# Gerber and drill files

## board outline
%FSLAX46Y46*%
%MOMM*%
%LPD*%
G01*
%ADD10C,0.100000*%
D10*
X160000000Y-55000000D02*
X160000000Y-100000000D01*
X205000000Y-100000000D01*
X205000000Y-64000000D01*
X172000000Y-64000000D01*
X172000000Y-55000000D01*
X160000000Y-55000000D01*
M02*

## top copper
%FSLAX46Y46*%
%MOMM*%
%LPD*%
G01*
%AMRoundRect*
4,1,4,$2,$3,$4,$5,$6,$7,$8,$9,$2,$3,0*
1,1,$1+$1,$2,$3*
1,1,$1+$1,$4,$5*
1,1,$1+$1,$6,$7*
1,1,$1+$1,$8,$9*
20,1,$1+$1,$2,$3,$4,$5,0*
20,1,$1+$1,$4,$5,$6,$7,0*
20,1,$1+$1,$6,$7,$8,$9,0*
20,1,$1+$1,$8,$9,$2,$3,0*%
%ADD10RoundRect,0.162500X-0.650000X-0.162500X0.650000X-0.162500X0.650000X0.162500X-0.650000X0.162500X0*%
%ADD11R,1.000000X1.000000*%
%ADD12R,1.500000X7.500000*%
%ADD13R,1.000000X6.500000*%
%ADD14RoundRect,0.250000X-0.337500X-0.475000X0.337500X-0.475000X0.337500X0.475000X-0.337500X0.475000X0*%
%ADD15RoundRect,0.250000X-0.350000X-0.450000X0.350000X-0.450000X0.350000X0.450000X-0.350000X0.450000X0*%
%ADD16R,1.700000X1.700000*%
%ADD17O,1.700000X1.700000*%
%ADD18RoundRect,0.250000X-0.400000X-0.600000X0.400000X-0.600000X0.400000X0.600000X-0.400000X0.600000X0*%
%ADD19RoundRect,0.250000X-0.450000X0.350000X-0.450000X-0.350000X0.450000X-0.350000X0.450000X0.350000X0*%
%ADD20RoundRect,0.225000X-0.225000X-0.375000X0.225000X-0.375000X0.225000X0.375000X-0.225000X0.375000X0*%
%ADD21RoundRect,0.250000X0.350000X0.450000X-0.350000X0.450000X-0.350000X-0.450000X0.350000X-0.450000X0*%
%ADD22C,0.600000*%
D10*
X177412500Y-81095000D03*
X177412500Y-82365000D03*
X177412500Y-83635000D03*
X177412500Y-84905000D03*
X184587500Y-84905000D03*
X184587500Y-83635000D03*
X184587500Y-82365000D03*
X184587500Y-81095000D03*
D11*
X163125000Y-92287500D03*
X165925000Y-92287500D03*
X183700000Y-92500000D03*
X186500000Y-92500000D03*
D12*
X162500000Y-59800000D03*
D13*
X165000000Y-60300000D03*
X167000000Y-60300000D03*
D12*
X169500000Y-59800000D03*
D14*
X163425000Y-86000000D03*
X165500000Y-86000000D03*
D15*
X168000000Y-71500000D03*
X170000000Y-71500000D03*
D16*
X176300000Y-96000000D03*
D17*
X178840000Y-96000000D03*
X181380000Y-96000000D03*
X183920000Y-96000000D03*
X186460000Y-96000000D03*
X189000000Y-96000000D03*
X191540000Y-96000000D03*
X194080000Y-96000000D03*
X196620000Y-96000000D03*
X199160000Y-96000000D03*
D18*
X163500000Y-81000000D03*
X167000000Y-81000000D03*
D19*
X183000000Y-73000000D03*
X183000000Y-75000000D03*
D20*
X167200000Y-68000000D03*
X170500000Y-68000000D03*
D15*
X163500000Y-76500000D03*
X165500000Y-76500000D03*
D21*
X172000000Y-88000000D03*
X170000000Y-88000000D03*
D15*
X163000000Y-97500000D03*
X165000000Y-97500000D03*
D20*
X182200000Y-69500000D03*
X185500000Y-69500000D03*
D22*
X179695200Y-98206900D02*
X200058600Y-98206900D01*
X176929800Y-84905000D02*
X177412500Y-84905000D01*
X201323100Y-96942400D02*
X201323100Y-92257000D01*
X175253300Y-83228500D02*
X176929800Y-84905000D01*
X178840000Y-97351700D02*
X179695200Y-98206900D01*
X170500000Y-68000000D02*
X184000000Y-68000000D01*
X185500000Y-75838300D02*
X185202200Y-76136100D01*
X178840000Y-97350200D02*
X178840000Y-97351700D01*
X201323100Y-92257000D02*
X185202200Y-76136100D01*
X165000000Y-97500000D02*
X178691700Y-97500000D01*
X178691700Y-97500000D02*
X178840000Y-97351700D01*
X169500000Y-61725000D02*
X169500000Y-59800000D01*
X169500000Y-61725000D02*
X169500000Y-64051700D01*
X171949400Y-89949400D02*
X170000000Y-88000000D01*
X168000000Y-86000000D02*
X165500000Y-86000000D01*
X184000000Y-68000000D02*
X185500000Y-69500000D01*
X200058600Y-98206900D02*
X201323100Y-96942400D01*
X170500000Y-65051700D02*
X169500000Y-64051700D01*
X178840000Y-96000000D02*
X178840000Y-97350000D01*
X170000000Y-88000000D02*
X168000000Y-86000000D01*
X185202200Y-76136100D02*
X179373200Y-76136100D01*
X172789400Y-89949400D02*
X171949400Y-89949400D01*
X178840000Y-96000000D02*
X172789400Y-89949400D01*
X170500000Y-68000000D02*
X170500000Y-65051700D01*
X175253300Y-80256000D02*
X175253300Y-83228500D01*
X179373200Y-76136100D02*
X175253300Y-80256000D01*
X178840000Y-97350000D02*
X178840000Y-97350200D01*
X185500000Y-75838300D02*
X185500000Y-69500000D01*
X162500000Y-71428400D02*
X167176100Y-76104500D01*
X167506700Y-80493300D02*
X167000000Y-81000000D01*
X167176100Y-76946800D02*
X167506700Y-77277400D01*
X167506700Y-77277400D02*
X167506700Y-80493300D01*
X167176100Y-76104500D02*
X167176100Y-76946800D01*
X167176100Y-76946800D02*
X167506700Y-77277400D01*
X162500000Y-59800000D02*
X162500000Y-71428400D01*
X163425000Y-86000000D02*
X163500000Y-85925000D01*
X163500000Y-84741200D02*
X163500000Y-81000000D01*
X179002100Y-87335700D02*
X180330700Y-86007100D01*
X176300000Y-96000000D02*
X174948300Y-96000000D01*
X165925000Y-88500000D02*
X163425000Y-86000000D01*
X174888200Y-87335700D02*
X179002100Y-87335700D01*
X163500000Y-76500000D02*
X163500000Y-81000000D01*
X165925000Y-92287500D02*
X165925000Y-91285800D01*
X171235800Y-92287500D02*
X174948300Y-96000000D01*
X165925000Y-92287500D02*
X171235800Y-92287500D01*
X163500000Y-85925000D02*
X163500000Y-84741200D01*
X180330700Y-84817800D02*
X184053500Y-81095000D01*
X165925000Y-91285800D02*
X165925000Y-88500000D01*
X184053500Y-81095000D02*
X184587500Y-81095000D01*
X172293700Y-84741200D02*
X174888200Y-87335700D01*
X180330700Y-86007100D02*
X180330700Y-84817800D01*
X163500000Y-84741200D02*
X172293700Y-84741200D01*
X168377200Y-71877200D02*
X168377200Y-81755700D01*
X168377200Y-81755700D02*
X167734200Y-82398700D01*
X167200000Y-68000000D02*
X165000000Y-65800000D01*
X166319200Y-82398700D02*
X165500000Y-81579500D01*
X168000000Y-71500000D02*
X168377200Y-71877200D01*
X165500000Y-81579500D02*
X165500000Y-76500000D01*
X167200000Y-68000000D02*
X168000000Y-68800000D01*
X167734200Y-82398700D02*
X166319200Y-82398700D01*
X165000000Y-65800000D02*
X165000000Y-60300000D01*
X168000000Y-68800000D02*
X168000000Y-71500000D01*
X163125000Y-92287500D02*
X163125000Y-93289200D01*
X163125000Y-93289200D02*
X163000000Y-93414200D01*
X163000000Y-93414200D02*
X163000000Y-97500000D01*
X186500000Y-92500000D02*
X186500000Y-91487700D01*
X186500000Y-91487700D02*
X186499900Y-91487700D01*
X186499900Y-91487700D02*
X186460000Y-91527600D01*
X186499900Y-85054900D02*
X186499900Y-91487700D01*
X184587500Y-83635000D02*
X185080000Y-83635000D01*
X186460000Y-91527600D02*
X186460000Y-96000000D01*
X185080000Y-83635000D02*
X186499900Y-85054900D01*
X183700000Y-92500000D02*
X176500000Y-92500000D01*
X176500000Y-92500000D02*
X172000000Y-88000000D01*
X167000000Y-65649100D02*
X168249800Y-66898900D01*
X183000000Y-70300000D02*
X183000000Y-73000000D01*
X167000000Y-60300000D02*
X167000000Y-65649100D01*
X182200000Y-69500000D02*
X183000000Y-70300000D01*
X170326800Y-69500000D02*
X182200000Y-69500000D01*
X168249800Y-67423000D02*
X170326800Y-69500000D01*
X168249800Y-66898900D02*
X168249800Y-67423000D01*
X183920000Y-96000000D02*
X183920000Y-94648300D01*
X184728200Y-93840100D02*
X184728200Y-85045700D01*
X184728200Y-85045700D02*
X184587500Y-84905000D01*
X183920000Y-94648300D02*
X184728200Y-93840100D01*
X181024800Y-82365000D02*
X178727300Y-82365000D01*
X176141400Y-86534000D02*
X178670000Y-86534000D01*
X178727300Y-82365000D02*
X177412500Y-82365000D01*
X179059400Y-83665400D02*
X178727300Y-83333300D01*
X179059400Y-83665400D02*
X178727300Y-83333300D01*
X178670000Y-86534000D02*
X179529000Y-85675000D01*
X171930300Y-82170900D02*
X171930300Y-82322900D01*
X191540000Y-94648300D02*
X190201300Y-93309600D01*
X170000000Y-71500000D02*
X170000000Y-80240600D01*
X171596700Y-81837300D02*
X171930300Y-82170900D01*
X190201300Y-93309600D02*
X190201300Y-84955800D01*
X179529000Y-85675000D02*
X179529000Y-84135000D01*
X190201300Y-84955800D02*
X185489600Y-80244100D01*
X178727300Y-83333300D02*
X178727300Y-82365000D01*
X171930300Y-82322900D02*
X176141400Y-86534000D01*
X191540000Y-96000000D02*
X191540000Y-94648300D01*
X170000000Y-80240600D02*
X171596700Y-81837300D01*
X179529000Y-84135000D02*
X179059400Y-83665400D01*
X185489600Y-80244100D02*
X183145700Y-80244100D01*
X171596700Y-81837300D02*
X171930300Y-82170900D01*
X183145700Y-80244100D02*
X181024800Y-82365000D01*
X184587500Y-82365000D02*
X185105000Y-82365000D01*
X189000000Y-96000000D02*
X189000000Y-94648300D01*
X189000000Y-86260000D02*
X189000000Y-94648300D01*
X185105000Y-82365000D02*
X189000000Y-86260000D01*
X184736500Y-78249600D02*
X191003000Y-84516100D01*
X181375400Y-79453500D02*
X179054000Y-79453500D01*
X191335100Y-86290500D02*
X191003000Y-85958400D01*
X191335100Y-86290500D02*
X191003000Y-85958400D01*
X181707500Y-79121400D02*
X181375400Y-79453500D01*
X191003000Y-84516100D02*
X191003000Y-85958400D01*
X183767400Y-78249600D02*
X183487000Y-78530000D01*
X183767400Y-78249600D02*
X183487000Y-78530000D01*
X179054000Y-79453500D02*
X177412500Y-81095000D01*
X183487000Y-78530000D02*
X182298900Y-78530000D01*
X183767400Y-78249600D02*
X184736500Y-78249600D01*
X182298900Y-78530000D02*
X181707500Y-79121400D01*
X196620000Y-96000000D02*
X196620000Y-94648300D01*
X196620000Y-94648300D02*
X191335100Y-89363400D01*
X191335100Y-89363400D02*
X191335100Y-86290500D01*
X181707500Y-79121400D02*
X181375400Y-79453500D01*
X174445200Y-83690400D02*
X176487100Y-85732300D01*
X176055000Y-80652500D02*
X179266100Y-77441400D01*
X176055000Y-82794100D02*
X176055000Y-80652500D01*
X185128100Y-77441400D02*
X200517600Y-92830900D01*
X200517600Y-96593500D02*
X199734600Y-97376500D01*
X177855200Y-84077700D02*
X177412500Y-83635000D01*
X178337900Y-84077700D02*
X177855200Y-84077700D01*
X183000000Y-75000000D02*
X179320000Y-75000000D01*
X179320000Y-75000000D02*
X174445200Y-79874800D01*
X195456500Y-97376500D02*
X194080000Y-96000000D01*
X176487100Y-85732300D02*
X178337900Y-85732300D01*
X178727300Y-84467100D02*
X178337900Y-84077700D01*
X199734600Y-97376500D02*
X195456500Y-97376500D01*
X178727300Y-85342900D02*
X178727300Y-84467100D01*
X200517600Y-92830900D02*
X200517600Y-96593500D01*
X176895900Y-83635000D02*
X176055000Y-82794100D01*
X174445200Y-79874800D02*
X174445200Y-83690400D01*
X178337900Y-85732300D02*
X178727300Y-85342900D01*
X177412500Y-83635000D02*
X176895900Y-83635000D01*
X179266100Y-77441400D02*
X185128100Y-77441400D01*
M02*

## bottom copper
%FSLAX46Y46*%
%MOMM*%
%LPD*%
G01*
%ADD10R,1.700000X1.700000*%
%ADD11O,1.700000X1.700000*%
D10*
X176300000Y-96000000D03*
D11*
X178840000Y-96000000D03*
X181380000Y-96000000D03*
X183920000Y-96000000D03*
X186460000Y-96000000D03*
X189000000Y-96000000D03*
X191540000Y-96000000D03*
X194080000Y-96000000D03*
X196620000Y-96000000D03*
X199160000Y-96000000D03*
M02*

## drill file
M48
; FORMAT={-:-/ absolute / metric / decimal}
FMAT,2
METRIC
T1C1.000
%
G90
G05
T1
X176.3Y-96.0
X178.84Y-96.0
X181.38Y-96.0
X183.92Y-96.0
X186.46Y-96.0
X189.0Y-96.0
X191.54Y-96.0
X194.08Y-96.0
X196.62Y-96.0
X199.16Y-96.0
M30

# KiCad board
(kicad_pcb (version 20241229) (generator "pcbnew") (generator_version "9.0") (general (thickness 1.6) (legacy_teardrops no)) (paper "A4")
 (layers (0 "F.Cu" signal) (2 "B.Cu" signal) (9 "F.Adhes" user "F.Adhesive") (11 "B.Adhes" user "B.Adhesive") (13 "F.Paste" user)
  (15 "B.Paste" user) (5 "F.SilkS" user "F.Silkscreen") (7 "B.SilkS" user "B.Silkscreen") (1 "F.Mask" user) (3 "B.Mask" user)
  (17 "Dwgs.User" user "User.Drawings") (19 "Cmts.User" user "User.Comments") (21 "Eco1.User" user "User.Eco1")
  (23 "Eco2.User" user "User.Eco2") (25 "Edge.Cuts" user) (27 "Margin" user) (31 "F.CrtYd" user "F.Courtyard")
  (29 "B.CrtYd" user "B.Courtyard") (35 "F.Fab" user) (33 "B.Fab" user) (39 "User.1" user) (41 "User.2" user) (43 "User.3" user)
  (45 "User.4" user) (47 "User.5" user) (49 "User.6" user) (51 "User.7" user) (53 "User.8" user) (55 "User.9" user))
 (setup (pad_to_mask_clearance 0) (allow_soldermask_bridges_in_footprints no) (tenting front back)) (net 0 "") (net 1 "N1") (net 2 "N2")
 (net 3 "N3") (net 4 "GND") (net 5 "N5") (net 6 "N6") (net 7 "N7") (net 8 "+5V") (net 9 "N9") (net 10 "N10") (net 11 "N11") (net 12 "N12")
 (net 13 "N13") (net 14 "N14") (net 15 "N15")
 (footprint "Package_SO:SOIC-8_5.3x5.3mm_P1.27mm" (layer "F.Cu") (at 181 83)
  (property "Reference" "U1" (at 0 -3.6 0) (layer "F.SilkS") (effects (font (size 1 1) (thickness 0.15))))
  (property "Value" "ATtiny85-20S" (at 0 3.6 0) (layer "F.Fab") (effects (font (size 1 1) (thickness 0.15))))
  (pad "1" smd roundrect (at -3.5875 -1.905) (size 1.625 0.65) (layers "F.Cu" "F.Mask" "F.Paste") (roundrect_rratio 0.25) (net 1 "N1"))
  (pad "2" smd roundrect (at -3.5875 -0.635) (size 1.625 0.65) (layers "F.Cu" "F.Mask" "F.Paste") (roundrect_rratio 0.25) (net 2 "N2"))
  (pad "3" smd roundrect (at -3.5875 0.635) (size 1.625 0.65) (layers "F.Cu" "F.Mask" "F.Paste") (roundrect_rratio 0.25) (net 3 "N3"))
  (pad "4" smd roundrect (at -3.5875 1.905) (size 1.625 0.65) (layers "F.Cu" "F.Mask" "F.Paste") (roundrect_rratio 0.25) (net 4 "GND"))
  (pad "5" smd roundrect (at 3.5875 1.905) (size 1.625 0.65) (layers "F.Cu" "F.Mask" "F.Paste") (roundrect_rratio 0.25) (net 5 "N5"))
  (pad "6" smd roundrect (at 3.5875 0.635) (size 1.625 0.65) (layers "F.Cu" "F.Mask" "F.Paste") (roundrect_rratio 0.25) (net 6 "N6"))
  (pad "7" smd roundrect (at 3.5875 -0.635) (size 1.625 0.65) (layers "F.Cu" "F.Mask" "F.Paste") (roundrect_rratio 0.25) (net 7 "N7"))
  (pad "8" smd roundrect (at 3.5875 -1.905) (size 1.625 0.65) (layers "F.Cu" "F.Mask" "F.Paste") (roundrect_rratio 0.25) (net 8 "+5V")))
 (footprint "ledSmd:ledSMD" (layer "F.Cu") (at 164.925 92.2875)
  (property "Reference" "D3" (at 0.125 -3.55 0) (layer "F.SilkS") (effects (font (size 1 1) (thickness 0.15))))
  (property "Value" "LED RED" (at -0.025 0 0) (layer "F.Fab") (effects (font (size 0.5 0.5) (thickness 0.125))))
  (pad "1" smd rect (at -1.8 0) (size 1 1) (layers "F.Cu" "F.Mask" "F.Paste") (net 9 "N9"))
  (pad "2" smd rect (at 1 0) (size 1 1) (layers "F.Cu" "F.Mask" "F.Paste") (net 8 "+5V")))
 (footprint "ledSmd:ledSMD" (layer "F.Cu") (at 185.5 92.5)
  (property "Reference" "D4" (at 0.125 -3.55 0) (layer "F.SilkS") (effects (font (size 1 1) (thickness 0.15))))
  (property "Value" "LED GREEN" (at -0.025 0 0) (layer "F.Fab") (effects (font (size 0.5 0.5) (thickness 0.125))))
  (pad "1" smd rect (at -1.8 0) (size 1 1) (layers "F.Cu" "F.Mask" "F.Paste") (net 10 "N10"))
  (pad "2" smd rect (at 1 0) (size 1 1) (layers "F.Cu" "F.Mask" "F.Paste") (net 6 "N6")))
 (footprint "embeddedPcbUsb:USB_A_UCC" (layer "F.Cu") (at 166 60 -90)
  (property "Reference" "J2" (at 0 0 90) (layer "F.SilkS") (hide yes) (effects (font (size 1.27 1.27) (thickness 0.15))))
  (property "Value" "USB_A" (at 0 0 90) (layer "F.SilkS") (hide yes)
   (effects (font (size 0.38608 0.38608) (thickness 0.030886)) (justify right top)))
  (pad "1" smd rect (at -0.2 3.5 270) (size 7.5 1.5) (layers "F.Cu" "F.Mask" "F.Paste") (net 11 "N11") (solder_mask_margin 0.1016))
  (pad "2" smd rect (at 0.3 1 270) (size 6.5 1) (layers "F.Cu" "F.Mask" "F.Paste") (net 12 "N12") (solder_mask_margin 0.1016))
  (pad "3" smd rect (at 0.3 -1 270) (size 6.5 1) (layers "F.Cu" "F.Mask" "F.Paste") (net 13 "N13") (solder_mask_margin 0.1016))
  (pad "4" smd rect (at -0.2 -3.5 270) (size 7.5 1.5) (layers "F.Cu" "F.Mask" "F.Paste") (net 4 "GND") (solder_mask_margin 0.1016)))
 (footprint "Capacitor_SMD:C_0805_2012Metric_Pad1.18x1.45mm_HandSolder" (layer "F.Cu") (at 164.4625 86)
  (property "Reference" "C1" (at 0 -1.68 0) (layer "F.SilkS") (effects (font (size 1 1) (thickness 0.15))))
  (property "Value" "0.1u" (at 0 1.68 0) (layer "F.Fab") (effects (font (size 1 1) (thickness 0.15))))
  (pad "1" smd roundrect (at -1.0375 0) (size 1.175 1.45) (layers "F.Cu" "F.Mask" "F.Paste") (roundrect_rratio 0.212766) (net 8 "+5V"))
  (pad "2" smd roundrect (at 1.0375 0) (size 1.175 1.45) (layers "F.Cu" "F.Mask" "F.Paste") (roundrect_rratio 0.212766) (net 4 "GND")))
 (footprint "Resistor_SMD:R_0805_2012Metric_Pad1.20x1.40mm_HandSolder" (layer "F.Cu") (at 169 71.5)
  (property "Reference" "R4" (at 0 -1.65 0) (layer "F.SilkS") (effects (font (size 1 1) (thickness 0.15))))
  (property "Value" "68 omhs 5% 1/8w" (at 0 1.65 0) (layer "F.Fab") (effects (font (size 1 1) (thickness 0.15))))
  (pad "1" smd roundrect (at -1 0) (size 1.2 1.4) (layers "F.Cu" "F.Mask" "F.Paste") (roundrect_rratio 0.208333) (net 12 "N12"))
  (pad "2" smd roundrect (at 1 0) (size 1.2 1.4) (layers "F.Cu" "F.Mask" "F.Paste") (roundrect_rratio 0.208333) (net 2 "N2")))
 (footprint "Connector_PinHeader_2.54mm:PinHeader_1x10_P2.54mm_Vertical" (layer "F.Cu") (at 176.3 96 90)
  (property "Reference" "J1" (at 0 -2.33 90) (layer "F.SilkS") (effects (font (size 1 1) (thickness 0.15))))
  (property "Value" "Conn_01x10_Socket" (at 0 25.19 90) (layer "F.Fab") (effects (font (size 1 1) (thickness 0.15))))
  (pad "1" thru_hole rect (at 0 0 90) (size 1.7 1.7) (drill 1) (layers "*.Cu" "*.Mask") (remove_unused_layers no) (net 8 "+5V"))
  (pad "2" thru_hole oval (at 0 2.54 90) (size 1.7 1.7) (drill 1) (layers "*.Cu" "*.Mask") (remove_unused_layers no) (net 4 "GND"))
  (pad "3" thru_hole oval (at 0 5.08 90) (size 1.7 1.7) (drill 1) (layers "*.Cu" "*.Mask") (remove_unused_layers no) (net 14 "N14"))
  (pad "4" thru_hole oval (at 0 7.62 90) (size 1.7 1.7) (drill 1) (layers "*.Cu" "*.Mask") (remove_unused_layers no) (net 5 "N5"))
  (pad "5" thru_hole oval (at 0 10.16 90) (size 1.7 1.7) (drill 1) (layers "*.Cu" "*.Mask") (remove_unused_layers no) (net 6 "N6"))
  (pad "6" thru_hole oval (at 0 12.7 90) (size 1.7 1.7) (drill 1) (layers "*.Cu" "*.Mask") (remove_unused_layers no) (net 7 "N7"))
  (pad "7" thru_hole oval (at 0 15.24 90) (size 1.7 1.7) (drill 1) (layers "*.Cu" "*.Mask") (remove_unused_layers no) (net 2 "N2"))
  (pad "8" thru_hole oval (at 0 17.78 90) (size 1.7 1.7) (drill 1) (layers "*.Cu" "*.Mask") (remove_unused_layers no) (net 3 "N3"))
  (pad "9" thru_hole oval (at 0 20.32 90) (size 1.7 1.7) (drill 1) (layers "*.Cu" "*.Mask") (remove_unused_layers no) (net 1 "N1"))
  (pad "10" thru_hole oval (at 0 22.86 90) (size 1.7 1.7) (drill 1) (layers "*.Cu" "*.Mask") (remove_unused_layers no) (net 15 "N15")))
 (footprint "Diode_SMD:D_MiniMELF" (layer "F.Cu") (at 165.25 81)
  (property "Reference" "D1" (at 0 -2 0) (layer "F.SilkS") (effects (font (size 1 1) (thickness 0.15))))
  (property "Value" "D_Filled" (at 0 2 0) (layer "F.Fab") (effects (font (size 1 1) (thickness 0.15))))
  (pad "1" smd roundrect (at -1.75 0) (size 1.3 1.7) (layers "F.Cu" "F.Mask" "F.Paste") (roundrect_rratio 0.1923076923) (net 8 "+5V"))
  (pad "2" smd roundrect (at 1.75 0) (size 1.3 1.7) (layers "F.Cu" "F.Mask" "F.Paste") (roundrect_rratio 0.1923076923) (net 11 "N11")))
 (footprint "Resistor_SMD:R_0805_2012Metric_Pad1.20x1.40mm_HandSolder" (layer "F.Cu") (at 183 74 -90)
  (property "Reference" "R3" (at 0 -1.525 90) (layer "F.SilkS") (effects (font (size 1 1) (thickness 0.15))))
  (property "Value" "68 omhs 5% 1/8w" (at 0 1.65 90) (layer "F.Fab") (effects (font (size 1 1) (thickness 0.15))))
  (pad "1" smd roundrect (at -1 0 270) (size 1.2 1.4) (layers "F.Cu" "F.Mask" "F.Paste") (roundrect_rratio 0.208333) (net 13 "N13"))
  (pad "2" smd roundrect (at 1 0 270) (size 1.2 1.4) (layers "F.Cu" "F.Mask" "F.Paste") (roundrect_rratio 0.208333) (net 3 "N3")))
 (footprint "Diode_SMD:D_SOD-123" (layer "F.Cu") (at 168.85 68)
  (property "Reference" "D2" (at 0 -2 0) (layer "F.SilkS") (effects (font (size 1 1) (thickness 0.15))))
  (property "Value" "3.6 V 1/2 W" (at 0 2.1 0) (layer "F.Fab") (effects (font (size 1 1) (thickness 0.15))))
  (pad "1" smd roundrect (at -1.65 0) (size 0.9 1.2) (layers "F.Cu" "F.Mask" "F.Paste") (roundrect_rratio 0.25) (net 12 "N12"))
  (pad "2" smd roundrect (at 1.65 0) (size 0.9 1.2) (layers "F.Cu" "F.Mask" "F.Paste") (roundrect_rratio 0.25) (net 4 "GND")))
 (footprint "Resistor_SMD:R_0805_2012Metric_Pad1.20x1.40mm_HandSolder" (layer "F.Cu") (at 164.5 76.5)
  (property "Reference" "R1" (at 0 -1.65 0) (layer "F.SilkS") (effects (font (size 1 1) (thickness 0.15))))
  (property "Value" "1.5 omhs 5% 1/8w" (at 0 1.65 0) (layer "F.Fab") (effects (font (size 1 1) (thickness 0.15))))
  (pad "1" smd roundrect (at -1 0) (size 1.2 1.4) (layers "F.Cu" "F.Mask" "F.Paste") (roundrect_rratio 0.208333) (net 8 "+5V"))
  (pad "2" smd roundrect (at 1 0) (size 1.2 1.4) (layers "F.Cu" "F.Mask" "F.Paste") (roundrect_rratio 0.208333) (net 12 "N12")))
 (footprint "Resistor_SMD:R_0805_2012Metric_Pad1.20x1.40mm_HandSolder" (layer "F.Cu") (at 171 88 180)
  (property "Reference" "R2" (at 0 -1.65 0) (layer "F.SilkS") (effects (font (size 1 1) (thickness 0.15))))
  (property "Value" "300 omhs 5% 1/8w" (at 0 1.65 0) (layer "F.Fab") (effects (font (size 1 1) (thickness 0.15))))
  (pad "1" smd roundrect (at -1 0 180) (size 1.2 1.4) (layers "F.Cu" "F.Mask" "F.Paste") (roundrect_rratio 0.208333) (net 10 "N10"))
  (pad "2" smd roundrect (at 1 0 180) (size 1.2 1.4) (layers "F.Cu" "F.Mask" "F.Paste") (roundrect_rratio 0.208333) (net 4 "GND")))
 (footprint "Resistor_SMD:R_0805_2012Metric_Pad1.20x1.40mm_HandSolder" (layer "F.Cu") (at 164 97.5)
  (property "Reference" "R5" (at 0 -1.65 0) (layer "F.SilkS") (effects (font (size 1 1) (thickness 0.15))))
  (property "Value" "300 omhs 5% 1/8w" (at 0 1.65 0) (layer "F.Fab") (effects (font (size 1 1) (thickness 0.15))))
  (pad "1" smd roundrect (at -1 0) (size 1.2 1.4) (layers "F.Cu" "F.Mask" "F.Paste") (roundrect_rratio 0.208333) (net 9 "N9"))
  (pad "2" smd roundrect (at 1 0) (size 1.2 1.4) (layers "F.Cu" "F.Mask" "F.Paste") (roundrect_rratio 0.208333) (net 4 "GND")))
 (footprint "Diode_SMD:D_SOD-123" (layer "F.Cu") (at 183.85 69.5)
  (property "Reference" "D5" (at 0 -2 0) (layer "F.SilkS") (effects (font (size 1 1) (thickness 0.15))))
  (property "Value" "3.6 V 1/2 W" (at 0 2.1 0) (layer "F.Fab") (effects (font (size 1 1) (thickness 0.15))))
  (pad "1" smd roundrect (at -1.65 0) (size 0.9 1.2) (layers "F.Cu" "F.Mask" "F.Paste") (roundrect_rratio 0.25) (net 13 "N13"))
  (pad "2" smd roundrect (at 1.65 0) (size 0.9 1.2) (layers "F.Cu" "F.Mask" "F.Paste") (roundrect_rratio 0.25) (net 4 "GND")))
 (gr_poly
  (pts (xy 160 55) (xy 160 100) (xy 205 100) (xy 205 64) (xy 172 64) (xy 172 55)) (stroke (width 0.1) (type solid)) (fill no)
  (layer "Edge.Cuts"))
 (segment (start 179.6952 98.2069) (end 200.0586 98.2069) (width 0.6) (layer "F.Cu") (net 4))
 (segment (start 176.9298 84.905) (end 177.4125 84.905) (width 0.6) (layer "F.Cu") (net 4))
 (segment (start 201.3231 96.9424) (end 201.3231 92.257) (width 0.6) (layer "F.Cu") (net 4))
 (segment (start 175.2533 83.2285) (end 176.9298 84.905) (width 0.6) (layer "F.Cu") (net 4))
 (segment (start 178.84 97.3517) (end 179.6952 98.2069) (width 0.6) (layer "F.Cu") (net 4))
 (segment (start 170.5 68) (end 184 68) (width 0.6) (layer "F.Cu") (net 4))
 (segment (start 185.5 75.8383) (end 185.2022 76.1361) (width 0.6) (layer "F.Cu") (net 4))
 (segment (start 178.84 97.3502) (end 178.84 97.3517) (width 0.6) (layer "F.Cu") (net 4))
 (segment (start 201.3231 92.257) (end 185.2022 76.1361) (width 0.6) (layer "F.Cu") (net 4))
 (segment (start 165 97.5) (end 178.6917 97.5) (width 0.6) (layer "F.Cu") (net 4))
 (segment (start 178.6917 97.5) (end 178.84 97.3517) (width 0.6) (layer "F.Cu") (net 4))
 (segment (start 169.5 61.725) (end 169.5 59.8) (width 0.6) (layer "F.Cu") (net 4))
 (segment (start 169.5 61.725) (end 169.5 64.0517) (width 0.6) (layer "F.Cu") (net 4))
 (segment (start 171.9494 89.9494) (end 170 88) (width 0.6) (layer "F.Cu") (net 4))
 (segment (start 168 86) (end 165.5 86) (width 0.6) (layer "F.Cu") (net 4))
 (segment (start 184 68) (end 185.5 69.5) (width 0.6) (layer "F.Cu") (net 4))
 (segment (start 200.0586 98.2069) (end 201.3231 96.9424) (width 0.6) (layer "F.Cu") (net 4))
 (segment (start 170.5 65.0517) (end 169.5 64.0517) (width 0.6) (layer "F.Cu") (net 4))
 (segment (start 178.84 96) (end 178.84 97.35) (width 0.6) (layer "F.Cu") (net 4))
 (segment (start 170 88) (end 168 86) (width 0.6) (layer "F.Cu") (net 4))
 (segment (start 185.2022 76.1361) (end 179.3732 76.1361) (width 0.6) (layer "F.Cu") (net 4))
 (segment (start 172.7894 89.9494) (end 171.9494 89.9494) (width 0.6) (layer "F.Cu") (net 4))
 (segment (start 178.84 96) (end 172.7894 89.9494) (width 0.6) (layer "F.Cu") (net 4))
 (segment (start 170.5 68) (end 170.5 65.0517) (width 0.6) (layer "F.Cu") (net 4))
 (segment (start 175.2533 80.256) (end 175.2533 83.2285) (width 0.6) (layer "F.Cu") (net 4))
 (segment (start 179.3732 76.1361) (end 175.2533 80.256) (width 0.6) (layer "F.Cu") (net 4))
 (segment (start 178.84 97.35) (end 178.84 97.3502) (width 0.6) (layer "F.Cu") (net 4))
 (segment (start 185.5 75.8383) (end 185.5 69.5) (width 0.6) (layer "F.Cu") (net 4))
 (segment (start 162.5 71.4284) (end 167.1761 76.1045) (width 0.6) (layer "F.Cu") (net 11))
 (segment (start 167.5067 80.4933) (end 167 81) (width 0.6) (layer "F.Cu") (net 11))
 (segment (start 167.1761 76.9468) (end 167.5067 77.2774) (width 0.6) (layer "F.Cu") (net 11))
 (segment (start 167.5067 77.2774) (end 167.5067 80.4933) (width 0.6) (layer "F.Cu") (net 11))
 (segment (start 167.1761 76.1045) (end 167.1761 76.9468) (width 0.6) (layer "F.Cu") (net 11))
 (segment (start 167.1761 76.9468) (end 167.5067 77.2774) (width 0.6) (layer "F.Cu") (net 11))
 (segment (start 162.5 59.8) (end 162.5 71.4284) (width 0.6) (layer "F.Cu") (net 11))
 (segment (start 163.425 86) (end 163.5 85.925) (width 0.6) (layer "F.Cu") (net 8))
 (segment (start 163.5 84.7412) (end 163.5 81) (width 0.6) (layer "F.Cu") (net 8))
 (segment (start 179.0021 87.3357) (end 180.3307 86.0071) (width 0.6) (layer "F.Cu") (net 8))
 (segment (start 176.3 96) (end 174.9483 96) (width 0.6) (layer "F.Cu") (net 8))
 (segment (start 165.925 88.5) (end 163.425 86) (width 0.6) (layer "F.Cu") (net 8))
 (segment (start 174.8882 87.3357) (end 179.0021 87.3357) (width 0.6) (layer "F.Cu") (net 8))
 (segment (start 163.5 76.5) (end 163.5 81) (width 0.6) (layer "F.Cu") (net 8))
 (segment (start 165.925 92.2875) (end 165.925 91.2858) (width 0.6) (layer "F.Cu") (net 8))
 (segment (start 171.2358 92.2875) (end 174.9483 96) (width 0.6) (layer "F.Cu") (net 8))
 (segment (start 165.925 92.2875) (end 171.2358 92.2875) (width 0.6) (layer "F.Cu") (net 8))
 (segment (start 163.5 85.925) (end 163.5 84.7412) (width 0.6) (layer "F.Cu") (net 8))
 (segment (start 180.3307 84.8178) (end 184.0535 81.095) (width 0.6) (layer "F.Cu") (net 8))
 (segment (start 165.925 91.2858) (end 165.925 88.5) (width 0.6) (layer "F.Cu") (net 8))
 (segment (start 184.0535 81.095) (end 184.5875 81.095) (width 0.6) (layer "F.Cu") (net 8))
 (segment (start 172.2937 84.7412) (end 174.8882 87.3357) (width 0.6) (layer "F.Cu") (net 8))
 (segment (start 180.3307 86.0071) (end 180.3307 84.8178) (width 0.6) (layer "F.Cu") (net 8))
 (segment (start 163.5 84.7412) (end 172.2937 84.7412) (width 0.6) (layer "F.Cu") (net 8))
 (segment (start 168.3772 71.8772) (end 168.3772 81.7557) (width 0.6) (layer "F.Cu") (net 12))
 (segment (start 168.3772 81.7557) (end 167.7342 82.3987) (width 0.6) (layer "F.Cu") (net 12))
 (segment (start 167.2 68) (end 165 65.8) (width 0.6) (layer "F.Cu") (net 12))
 (segment (start 166.3192 82.3987) (end 165.5 81.5795) (width 0.6) (layer "F.Cu") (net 12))
 (segment (start 168 71.5) (end 168.3772 71.8772) (width 0.6) (layer "F.Cu") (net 12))
 (segment (start 165.5 81.5795) (end 165.5 76.5) (width 0.6) (layer "F.Cu") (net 12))
 (segment (start 167.2 68) (end 168 68.8) (width 0.6) (layer "F.Cu") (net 12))
 (segment (start 167.7342 82.3987) (end 166.3192 82.3987) (width 0.6) (layer "F.Cu") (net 12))
 (segment (start 165 65.8) (end 165 60.3) (width 0.6) (layer "F.Cu") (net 12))
 (segment (start 168 68.8) (end 168 71.5) (width 0.6) (layer "F.Cu") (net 12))
 (segment (start 163.125 92.2875) (end 163.125 93.2892) (width 0.6) (layer "F.Cu") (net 9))
 (segment (start 163.125 93.2892) (end 163 93.4142) (width 0.6) (layer "F.Cu") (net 9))
 (segment (start 163 93.4142) (end 163 97.5) (width 0.6) (layer "F.Cu") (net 9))
 (segment (start 186.5 92.5) (end 186.5 91.4877) (width 0.6) (layer "F.Cu") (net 6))
 (segment (start 186.5 91.4877) (end 186.4999 91.4877) (width 0.6) (layer "F.Cu") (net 6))
 (segment (start 186.4999 91.4877) (end 186.46 91.5276) (width 0.6) (layer "F.Cu") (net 6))
 (segment (start 186.4999 85.0549) (end 186.4999 91.4877) (width 0.6) (layer "F.Cu") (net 6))
 (segment (start 184.5875 83.635) (end 185.08 83.635) (width 0.6) (layer "F.Cu") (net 6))
 (segment (start 186.46 91.5276) (end 186.46 96) (width 0.6) (layer "F.Cu") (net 6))
 (segment (start 185.08 83.635) (end 186.4999 85.0549) (width 0.6) (layer "F.Cu") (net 6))
 (segment (start 183.7 92.5) (end 176.5 92.5) (width 0.6) (layer "F.Cu") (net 10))
 (segment (start 176.5 92.5) (end 172 88) (width 0.6) (layer "F.Cu") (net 10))
 (segment (start 167 65.6491) (end 168.2498 66.8989) (width 0.6) (layer "F.Cu") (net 13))
 (segment (start 183 70.3) (end 183 73) (width 0.6) (layer "F.Cu") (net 13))
 (segment (start 167 60.3) (end 167 65.6491) (width 0.6) (layer "F.Cu") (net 13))
 (segment (start 182.2 69.5) (end 183 70.3) (width 0.6) (layer "F.Cu") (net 13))
 (segment (start 170.3268 69.5) (end 182.2 69.5) (width 0.6) (layer "F.Cu") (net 13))
 (segment (start 168.2498 67.423) (end 170.3268 69.5) (width 0.6) (layer "F.Cu") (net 13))
 (segment (start 168.2498 66.8989) (end 168.2498 67.423) (width 0.6) (layer "F.Cu") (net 13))
 (segment (start 183.92 96) (end 183.92 94.6483) (width 0.6) (layer "F.Cu") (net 5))
 (segment (start 184.7282 93.8401) (end 184.7282 85.0457) (width 0.6) (layer "F.Cu") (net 5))
 (segment (start 184.7282 85.0457) (end 184.5875 84.905) (width 0.6) (layer "F.Cu") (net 5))
 (segment (start 183.92 94.6483) (end 184.7282 93.8401) (width 0.6) (layer "F.Cu") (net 5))
 (segment (start 181.0248 82.365) (end 178.7273 82.365) (width 0.6) (layer "F.Cu") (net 2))
 (segment (start 176.1414 86.534) (end 178.67 86.534) (width 0.6) (layer "F.Cu") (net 2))
 (segment (start 178.7273 82.365) (end 177.4125 82.365) (width 0.6) (layer "F.Cu") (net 2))
 (segment (start 179.0594 83.6654) (end 178.7273 83.3333) (width 0.6) (layer "F.Cu") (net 2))
 (segment (start 179.0594 83.6654) (end 178.7273 83.3333) (width 0.6) (layer "F.Cu") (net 2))
 (segment (start 178.67 86.534) (end 179.529 85.675) (width 0.6) (layer "F.Cu") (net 2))
 (segment (start 171.9303 82.1709) (end 171.9303 82.3229) (width 0.6) (layer "F.Cu") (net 2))
 (segment (start 191.54 94.6483) (end 190.2013 93.3096) (width 0.6) (layer "F.Cu") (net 2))
 (segment (start 170 71.5) (end 170 80.2406) (width 0.6) (layer "F.Cu") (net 2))
 (segment (start 171.5967 81.8373) (end 171.9303 82.1709) (width 0.6) (layer "F.Cu") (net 2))
 (segment (start 190.2013 93.3096) (end 190.2013 84.9558) (width 0.6) (layer "F.Cu") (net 2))
 (segment (start 179.529 85.675) (end 179.529 84.135) (width 0.6) (layer "F.Cu") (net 2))
 (segment (start 190.2013 84.9558) (end 185.4896 80.2441) (width 0.6) (layer "F.Cu") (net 2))
 (segment (start 178.7273 83.3333) (end 178.7273 82.365) (width 0.6) (layer "F.Cu") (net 2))
 (segment (start 171.9303 82.3229) (end 176.1414 86.534) (width 0.6) (layer "F.Cu") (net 2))
 (segment (start 191.54 96) (end 191.54 94.6483) (width 0.6) (layer "F.Cu") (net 2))
 (segment (start 170 80.2406) (end 171.5967 81.8373) (width 0.6) (layer "F.Cu") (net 2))
 (segment (start 179.529 84.135) (end 179.0594 83.6654) (width 0.6) (layer "F.Cu") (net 2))
 (segment (start 185.4896 80.2441) (end 183.1457 80.2441) (width 0.6) (layer "F.Cu") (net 2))
 (segment (start 171.5967 81.8373) (end 171.9303 82.1709) (width 0.6) (layer "F.Cu") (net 2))
 (segment (start 183.1457 80.2441) (end 181.0248 82.365) (width 0.6) (layer "F.Cu") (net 2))
 (segment (start 184.5875 82.365) (end 185.105 82.365) (width 0.6) (layer "F.Cu") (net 7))
 (segment (start 189 96) (end 189 94.6483) (width 0.6) (layer "F.Cu") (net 7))
 (segment (start 189 86.26) (end 189 94.6483) (width 0.6) (layer "F.Cu") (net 7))
 (segment (start 185.105 82.365) (end 189 86.26) (width 0.6) (layer "F.Cu") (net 7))
 (segment (start 184.7365 78.2496) (end 191.003 84.5161) (width 0.6) (layer "F.Cu") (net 1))
 (segment (start 181.3754 79.4535) (end 179.054 79.4535) (width 0.6) (layer "F.Cu") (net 1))
 (segment (start 191.3351 86.2905) (end 191.003 85.9584) (width 0.6) (layer "F.Cu") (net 1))
 (segment (start 191.3351 86.2905) (end 191.003 85.9584) (width 0.6) (layer "F.Cu") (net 1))
 (segment (start 181.7075 79.1214) (end 181.3754 79.4535) (width 0.6) (layer "F.Cu") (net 1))
 (segment (start 191.003 84.5161) (end 191.003 85.9584) (width 0.6) (layer "F.Cu") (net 1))
 (segment (start 183.7674 78.2496) (end 183.487 78.53) (width 0.6) (layer "F.Cu") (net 1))
 (segment (start 183.7674 78.2496) (end 183.487 78.53) (width 0.6) (layer "F.Cu") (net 1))
 (segment (start 179.054 79.4535) (end 177.4125 81.095) (width 0.6) (layer "F.Cu") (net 1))
 (segment (start 183.487 78.53) (end 182.2989 78.53) (width 0.6) (layer "F.Cu") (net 1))
 (segment (start 183.7674 78.2496) (end 184.7365 78.2496) (width 0.6) (layer "F.Cu") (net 1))
 (segment (start 182.2989 78.53) (end 181.7075 79.1214) (width 0.6) (layer "F.Cu") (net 1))
 (segment (start 196.62 96) (end 196.62 94.6483) (width 0.6) (layer "F.Cu") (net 1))
 (segment (start 196.62 94.6483) (end 191.3351 89.3634) (width 0.6) (layer "F.Cu") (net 1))
 (segment (start 191.3351 89.3634) (end 191.3351 86.2905) (width 0.6) (layer "F.Cu") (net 1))
 (segment (start 181.7075 79.1214) (end 181.3754 79.4535) (width 0.6) (layer "F.Cu") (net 1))
 (segment (start 174.4452 83.6904) (end 176.4871 85.7323) (width 0.6) (layer "F.Cu") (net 3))
 (segment (start 176.055 80.6525) (end 179.2661 77.4414) (width 0.6) (layer "F.Cu") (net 3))
 (segment (start 176.055 82.7941) (end 176.055 80.6525) (width 0.6) (layer "F.Cu") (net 3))
 (segment (start 185.1281 77.4414) (end 200.5176 92.8309) (width 0.6) (layer "F.Cu") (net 3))
 (segment (start 200.5176 96.5935) (end 199.7346 97.3765) (width 0.6) (layer "F.Cu") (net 3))
 (segment (start 177.8552 84.0777) (end 177.4125 83.635) (width 0.6) (layer "F.Cu") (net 3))
 (segment (start 178.3379 84.0777) (end 177.8552 84.0777) (width 0.6) (layer "F.Cu") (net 3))
 (segment (start 183 75) (end 179.32 75) (width 0.6) (layer "F.Cu") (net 3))
 (segment (start 179.32 75) (end 174.4452 79.8748) (width 0.6) (layer "F.Cu") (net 3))
 (segment (start 195.4565 97.3765) (end 194.08 96) (width 0.6) (layer "F.Cu") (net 3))
 (segment (start 176.4871 85.7323) (end 178.3379 85.7323) (width 0.6) (layer "F.Cu") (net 3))
 (segment (start 178.7273 84.4671) (end 178.3379 84.0777) (width 0.6) (layer "F.Cu") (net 3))
 (segment (start 199.7346 97.3765) (end 195.4565 97.3765) (width 0.6) (layer "F.Cu") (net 3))
 (segment (start 178.7273 85.3429) (end 178.7273 84.4671) (width 0.6) (layer "F.Cu") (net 3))
 (segment (start 200.5176 92.8309) (end 200.5176 96.5935) (width 0.6) (layer "F.Cu") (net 3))
 (segment (start 176.8959 83.635) (end 176.055 82.7941) (width 0.6) (layer "F.Cu") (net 3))
 (segment (start 174.4452 79.8748) (end 174.4452 83.6904) (width 0.6) (layer "F.Cu") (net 3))
 (segment (start 178.3379 85.7323) (end 178.7273 85.3429) (width 0.6) (layer "F.Cu") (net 3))
 (segment (start 177.4125 83.635) (end 176.8959 83.635) (width 0.6) (layer "F.Cu") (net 3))
 (segment (start 179.2661 77.4414) (end 185.1281 77.4414) (width 0.6) (layer "F.Cu") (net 3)))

